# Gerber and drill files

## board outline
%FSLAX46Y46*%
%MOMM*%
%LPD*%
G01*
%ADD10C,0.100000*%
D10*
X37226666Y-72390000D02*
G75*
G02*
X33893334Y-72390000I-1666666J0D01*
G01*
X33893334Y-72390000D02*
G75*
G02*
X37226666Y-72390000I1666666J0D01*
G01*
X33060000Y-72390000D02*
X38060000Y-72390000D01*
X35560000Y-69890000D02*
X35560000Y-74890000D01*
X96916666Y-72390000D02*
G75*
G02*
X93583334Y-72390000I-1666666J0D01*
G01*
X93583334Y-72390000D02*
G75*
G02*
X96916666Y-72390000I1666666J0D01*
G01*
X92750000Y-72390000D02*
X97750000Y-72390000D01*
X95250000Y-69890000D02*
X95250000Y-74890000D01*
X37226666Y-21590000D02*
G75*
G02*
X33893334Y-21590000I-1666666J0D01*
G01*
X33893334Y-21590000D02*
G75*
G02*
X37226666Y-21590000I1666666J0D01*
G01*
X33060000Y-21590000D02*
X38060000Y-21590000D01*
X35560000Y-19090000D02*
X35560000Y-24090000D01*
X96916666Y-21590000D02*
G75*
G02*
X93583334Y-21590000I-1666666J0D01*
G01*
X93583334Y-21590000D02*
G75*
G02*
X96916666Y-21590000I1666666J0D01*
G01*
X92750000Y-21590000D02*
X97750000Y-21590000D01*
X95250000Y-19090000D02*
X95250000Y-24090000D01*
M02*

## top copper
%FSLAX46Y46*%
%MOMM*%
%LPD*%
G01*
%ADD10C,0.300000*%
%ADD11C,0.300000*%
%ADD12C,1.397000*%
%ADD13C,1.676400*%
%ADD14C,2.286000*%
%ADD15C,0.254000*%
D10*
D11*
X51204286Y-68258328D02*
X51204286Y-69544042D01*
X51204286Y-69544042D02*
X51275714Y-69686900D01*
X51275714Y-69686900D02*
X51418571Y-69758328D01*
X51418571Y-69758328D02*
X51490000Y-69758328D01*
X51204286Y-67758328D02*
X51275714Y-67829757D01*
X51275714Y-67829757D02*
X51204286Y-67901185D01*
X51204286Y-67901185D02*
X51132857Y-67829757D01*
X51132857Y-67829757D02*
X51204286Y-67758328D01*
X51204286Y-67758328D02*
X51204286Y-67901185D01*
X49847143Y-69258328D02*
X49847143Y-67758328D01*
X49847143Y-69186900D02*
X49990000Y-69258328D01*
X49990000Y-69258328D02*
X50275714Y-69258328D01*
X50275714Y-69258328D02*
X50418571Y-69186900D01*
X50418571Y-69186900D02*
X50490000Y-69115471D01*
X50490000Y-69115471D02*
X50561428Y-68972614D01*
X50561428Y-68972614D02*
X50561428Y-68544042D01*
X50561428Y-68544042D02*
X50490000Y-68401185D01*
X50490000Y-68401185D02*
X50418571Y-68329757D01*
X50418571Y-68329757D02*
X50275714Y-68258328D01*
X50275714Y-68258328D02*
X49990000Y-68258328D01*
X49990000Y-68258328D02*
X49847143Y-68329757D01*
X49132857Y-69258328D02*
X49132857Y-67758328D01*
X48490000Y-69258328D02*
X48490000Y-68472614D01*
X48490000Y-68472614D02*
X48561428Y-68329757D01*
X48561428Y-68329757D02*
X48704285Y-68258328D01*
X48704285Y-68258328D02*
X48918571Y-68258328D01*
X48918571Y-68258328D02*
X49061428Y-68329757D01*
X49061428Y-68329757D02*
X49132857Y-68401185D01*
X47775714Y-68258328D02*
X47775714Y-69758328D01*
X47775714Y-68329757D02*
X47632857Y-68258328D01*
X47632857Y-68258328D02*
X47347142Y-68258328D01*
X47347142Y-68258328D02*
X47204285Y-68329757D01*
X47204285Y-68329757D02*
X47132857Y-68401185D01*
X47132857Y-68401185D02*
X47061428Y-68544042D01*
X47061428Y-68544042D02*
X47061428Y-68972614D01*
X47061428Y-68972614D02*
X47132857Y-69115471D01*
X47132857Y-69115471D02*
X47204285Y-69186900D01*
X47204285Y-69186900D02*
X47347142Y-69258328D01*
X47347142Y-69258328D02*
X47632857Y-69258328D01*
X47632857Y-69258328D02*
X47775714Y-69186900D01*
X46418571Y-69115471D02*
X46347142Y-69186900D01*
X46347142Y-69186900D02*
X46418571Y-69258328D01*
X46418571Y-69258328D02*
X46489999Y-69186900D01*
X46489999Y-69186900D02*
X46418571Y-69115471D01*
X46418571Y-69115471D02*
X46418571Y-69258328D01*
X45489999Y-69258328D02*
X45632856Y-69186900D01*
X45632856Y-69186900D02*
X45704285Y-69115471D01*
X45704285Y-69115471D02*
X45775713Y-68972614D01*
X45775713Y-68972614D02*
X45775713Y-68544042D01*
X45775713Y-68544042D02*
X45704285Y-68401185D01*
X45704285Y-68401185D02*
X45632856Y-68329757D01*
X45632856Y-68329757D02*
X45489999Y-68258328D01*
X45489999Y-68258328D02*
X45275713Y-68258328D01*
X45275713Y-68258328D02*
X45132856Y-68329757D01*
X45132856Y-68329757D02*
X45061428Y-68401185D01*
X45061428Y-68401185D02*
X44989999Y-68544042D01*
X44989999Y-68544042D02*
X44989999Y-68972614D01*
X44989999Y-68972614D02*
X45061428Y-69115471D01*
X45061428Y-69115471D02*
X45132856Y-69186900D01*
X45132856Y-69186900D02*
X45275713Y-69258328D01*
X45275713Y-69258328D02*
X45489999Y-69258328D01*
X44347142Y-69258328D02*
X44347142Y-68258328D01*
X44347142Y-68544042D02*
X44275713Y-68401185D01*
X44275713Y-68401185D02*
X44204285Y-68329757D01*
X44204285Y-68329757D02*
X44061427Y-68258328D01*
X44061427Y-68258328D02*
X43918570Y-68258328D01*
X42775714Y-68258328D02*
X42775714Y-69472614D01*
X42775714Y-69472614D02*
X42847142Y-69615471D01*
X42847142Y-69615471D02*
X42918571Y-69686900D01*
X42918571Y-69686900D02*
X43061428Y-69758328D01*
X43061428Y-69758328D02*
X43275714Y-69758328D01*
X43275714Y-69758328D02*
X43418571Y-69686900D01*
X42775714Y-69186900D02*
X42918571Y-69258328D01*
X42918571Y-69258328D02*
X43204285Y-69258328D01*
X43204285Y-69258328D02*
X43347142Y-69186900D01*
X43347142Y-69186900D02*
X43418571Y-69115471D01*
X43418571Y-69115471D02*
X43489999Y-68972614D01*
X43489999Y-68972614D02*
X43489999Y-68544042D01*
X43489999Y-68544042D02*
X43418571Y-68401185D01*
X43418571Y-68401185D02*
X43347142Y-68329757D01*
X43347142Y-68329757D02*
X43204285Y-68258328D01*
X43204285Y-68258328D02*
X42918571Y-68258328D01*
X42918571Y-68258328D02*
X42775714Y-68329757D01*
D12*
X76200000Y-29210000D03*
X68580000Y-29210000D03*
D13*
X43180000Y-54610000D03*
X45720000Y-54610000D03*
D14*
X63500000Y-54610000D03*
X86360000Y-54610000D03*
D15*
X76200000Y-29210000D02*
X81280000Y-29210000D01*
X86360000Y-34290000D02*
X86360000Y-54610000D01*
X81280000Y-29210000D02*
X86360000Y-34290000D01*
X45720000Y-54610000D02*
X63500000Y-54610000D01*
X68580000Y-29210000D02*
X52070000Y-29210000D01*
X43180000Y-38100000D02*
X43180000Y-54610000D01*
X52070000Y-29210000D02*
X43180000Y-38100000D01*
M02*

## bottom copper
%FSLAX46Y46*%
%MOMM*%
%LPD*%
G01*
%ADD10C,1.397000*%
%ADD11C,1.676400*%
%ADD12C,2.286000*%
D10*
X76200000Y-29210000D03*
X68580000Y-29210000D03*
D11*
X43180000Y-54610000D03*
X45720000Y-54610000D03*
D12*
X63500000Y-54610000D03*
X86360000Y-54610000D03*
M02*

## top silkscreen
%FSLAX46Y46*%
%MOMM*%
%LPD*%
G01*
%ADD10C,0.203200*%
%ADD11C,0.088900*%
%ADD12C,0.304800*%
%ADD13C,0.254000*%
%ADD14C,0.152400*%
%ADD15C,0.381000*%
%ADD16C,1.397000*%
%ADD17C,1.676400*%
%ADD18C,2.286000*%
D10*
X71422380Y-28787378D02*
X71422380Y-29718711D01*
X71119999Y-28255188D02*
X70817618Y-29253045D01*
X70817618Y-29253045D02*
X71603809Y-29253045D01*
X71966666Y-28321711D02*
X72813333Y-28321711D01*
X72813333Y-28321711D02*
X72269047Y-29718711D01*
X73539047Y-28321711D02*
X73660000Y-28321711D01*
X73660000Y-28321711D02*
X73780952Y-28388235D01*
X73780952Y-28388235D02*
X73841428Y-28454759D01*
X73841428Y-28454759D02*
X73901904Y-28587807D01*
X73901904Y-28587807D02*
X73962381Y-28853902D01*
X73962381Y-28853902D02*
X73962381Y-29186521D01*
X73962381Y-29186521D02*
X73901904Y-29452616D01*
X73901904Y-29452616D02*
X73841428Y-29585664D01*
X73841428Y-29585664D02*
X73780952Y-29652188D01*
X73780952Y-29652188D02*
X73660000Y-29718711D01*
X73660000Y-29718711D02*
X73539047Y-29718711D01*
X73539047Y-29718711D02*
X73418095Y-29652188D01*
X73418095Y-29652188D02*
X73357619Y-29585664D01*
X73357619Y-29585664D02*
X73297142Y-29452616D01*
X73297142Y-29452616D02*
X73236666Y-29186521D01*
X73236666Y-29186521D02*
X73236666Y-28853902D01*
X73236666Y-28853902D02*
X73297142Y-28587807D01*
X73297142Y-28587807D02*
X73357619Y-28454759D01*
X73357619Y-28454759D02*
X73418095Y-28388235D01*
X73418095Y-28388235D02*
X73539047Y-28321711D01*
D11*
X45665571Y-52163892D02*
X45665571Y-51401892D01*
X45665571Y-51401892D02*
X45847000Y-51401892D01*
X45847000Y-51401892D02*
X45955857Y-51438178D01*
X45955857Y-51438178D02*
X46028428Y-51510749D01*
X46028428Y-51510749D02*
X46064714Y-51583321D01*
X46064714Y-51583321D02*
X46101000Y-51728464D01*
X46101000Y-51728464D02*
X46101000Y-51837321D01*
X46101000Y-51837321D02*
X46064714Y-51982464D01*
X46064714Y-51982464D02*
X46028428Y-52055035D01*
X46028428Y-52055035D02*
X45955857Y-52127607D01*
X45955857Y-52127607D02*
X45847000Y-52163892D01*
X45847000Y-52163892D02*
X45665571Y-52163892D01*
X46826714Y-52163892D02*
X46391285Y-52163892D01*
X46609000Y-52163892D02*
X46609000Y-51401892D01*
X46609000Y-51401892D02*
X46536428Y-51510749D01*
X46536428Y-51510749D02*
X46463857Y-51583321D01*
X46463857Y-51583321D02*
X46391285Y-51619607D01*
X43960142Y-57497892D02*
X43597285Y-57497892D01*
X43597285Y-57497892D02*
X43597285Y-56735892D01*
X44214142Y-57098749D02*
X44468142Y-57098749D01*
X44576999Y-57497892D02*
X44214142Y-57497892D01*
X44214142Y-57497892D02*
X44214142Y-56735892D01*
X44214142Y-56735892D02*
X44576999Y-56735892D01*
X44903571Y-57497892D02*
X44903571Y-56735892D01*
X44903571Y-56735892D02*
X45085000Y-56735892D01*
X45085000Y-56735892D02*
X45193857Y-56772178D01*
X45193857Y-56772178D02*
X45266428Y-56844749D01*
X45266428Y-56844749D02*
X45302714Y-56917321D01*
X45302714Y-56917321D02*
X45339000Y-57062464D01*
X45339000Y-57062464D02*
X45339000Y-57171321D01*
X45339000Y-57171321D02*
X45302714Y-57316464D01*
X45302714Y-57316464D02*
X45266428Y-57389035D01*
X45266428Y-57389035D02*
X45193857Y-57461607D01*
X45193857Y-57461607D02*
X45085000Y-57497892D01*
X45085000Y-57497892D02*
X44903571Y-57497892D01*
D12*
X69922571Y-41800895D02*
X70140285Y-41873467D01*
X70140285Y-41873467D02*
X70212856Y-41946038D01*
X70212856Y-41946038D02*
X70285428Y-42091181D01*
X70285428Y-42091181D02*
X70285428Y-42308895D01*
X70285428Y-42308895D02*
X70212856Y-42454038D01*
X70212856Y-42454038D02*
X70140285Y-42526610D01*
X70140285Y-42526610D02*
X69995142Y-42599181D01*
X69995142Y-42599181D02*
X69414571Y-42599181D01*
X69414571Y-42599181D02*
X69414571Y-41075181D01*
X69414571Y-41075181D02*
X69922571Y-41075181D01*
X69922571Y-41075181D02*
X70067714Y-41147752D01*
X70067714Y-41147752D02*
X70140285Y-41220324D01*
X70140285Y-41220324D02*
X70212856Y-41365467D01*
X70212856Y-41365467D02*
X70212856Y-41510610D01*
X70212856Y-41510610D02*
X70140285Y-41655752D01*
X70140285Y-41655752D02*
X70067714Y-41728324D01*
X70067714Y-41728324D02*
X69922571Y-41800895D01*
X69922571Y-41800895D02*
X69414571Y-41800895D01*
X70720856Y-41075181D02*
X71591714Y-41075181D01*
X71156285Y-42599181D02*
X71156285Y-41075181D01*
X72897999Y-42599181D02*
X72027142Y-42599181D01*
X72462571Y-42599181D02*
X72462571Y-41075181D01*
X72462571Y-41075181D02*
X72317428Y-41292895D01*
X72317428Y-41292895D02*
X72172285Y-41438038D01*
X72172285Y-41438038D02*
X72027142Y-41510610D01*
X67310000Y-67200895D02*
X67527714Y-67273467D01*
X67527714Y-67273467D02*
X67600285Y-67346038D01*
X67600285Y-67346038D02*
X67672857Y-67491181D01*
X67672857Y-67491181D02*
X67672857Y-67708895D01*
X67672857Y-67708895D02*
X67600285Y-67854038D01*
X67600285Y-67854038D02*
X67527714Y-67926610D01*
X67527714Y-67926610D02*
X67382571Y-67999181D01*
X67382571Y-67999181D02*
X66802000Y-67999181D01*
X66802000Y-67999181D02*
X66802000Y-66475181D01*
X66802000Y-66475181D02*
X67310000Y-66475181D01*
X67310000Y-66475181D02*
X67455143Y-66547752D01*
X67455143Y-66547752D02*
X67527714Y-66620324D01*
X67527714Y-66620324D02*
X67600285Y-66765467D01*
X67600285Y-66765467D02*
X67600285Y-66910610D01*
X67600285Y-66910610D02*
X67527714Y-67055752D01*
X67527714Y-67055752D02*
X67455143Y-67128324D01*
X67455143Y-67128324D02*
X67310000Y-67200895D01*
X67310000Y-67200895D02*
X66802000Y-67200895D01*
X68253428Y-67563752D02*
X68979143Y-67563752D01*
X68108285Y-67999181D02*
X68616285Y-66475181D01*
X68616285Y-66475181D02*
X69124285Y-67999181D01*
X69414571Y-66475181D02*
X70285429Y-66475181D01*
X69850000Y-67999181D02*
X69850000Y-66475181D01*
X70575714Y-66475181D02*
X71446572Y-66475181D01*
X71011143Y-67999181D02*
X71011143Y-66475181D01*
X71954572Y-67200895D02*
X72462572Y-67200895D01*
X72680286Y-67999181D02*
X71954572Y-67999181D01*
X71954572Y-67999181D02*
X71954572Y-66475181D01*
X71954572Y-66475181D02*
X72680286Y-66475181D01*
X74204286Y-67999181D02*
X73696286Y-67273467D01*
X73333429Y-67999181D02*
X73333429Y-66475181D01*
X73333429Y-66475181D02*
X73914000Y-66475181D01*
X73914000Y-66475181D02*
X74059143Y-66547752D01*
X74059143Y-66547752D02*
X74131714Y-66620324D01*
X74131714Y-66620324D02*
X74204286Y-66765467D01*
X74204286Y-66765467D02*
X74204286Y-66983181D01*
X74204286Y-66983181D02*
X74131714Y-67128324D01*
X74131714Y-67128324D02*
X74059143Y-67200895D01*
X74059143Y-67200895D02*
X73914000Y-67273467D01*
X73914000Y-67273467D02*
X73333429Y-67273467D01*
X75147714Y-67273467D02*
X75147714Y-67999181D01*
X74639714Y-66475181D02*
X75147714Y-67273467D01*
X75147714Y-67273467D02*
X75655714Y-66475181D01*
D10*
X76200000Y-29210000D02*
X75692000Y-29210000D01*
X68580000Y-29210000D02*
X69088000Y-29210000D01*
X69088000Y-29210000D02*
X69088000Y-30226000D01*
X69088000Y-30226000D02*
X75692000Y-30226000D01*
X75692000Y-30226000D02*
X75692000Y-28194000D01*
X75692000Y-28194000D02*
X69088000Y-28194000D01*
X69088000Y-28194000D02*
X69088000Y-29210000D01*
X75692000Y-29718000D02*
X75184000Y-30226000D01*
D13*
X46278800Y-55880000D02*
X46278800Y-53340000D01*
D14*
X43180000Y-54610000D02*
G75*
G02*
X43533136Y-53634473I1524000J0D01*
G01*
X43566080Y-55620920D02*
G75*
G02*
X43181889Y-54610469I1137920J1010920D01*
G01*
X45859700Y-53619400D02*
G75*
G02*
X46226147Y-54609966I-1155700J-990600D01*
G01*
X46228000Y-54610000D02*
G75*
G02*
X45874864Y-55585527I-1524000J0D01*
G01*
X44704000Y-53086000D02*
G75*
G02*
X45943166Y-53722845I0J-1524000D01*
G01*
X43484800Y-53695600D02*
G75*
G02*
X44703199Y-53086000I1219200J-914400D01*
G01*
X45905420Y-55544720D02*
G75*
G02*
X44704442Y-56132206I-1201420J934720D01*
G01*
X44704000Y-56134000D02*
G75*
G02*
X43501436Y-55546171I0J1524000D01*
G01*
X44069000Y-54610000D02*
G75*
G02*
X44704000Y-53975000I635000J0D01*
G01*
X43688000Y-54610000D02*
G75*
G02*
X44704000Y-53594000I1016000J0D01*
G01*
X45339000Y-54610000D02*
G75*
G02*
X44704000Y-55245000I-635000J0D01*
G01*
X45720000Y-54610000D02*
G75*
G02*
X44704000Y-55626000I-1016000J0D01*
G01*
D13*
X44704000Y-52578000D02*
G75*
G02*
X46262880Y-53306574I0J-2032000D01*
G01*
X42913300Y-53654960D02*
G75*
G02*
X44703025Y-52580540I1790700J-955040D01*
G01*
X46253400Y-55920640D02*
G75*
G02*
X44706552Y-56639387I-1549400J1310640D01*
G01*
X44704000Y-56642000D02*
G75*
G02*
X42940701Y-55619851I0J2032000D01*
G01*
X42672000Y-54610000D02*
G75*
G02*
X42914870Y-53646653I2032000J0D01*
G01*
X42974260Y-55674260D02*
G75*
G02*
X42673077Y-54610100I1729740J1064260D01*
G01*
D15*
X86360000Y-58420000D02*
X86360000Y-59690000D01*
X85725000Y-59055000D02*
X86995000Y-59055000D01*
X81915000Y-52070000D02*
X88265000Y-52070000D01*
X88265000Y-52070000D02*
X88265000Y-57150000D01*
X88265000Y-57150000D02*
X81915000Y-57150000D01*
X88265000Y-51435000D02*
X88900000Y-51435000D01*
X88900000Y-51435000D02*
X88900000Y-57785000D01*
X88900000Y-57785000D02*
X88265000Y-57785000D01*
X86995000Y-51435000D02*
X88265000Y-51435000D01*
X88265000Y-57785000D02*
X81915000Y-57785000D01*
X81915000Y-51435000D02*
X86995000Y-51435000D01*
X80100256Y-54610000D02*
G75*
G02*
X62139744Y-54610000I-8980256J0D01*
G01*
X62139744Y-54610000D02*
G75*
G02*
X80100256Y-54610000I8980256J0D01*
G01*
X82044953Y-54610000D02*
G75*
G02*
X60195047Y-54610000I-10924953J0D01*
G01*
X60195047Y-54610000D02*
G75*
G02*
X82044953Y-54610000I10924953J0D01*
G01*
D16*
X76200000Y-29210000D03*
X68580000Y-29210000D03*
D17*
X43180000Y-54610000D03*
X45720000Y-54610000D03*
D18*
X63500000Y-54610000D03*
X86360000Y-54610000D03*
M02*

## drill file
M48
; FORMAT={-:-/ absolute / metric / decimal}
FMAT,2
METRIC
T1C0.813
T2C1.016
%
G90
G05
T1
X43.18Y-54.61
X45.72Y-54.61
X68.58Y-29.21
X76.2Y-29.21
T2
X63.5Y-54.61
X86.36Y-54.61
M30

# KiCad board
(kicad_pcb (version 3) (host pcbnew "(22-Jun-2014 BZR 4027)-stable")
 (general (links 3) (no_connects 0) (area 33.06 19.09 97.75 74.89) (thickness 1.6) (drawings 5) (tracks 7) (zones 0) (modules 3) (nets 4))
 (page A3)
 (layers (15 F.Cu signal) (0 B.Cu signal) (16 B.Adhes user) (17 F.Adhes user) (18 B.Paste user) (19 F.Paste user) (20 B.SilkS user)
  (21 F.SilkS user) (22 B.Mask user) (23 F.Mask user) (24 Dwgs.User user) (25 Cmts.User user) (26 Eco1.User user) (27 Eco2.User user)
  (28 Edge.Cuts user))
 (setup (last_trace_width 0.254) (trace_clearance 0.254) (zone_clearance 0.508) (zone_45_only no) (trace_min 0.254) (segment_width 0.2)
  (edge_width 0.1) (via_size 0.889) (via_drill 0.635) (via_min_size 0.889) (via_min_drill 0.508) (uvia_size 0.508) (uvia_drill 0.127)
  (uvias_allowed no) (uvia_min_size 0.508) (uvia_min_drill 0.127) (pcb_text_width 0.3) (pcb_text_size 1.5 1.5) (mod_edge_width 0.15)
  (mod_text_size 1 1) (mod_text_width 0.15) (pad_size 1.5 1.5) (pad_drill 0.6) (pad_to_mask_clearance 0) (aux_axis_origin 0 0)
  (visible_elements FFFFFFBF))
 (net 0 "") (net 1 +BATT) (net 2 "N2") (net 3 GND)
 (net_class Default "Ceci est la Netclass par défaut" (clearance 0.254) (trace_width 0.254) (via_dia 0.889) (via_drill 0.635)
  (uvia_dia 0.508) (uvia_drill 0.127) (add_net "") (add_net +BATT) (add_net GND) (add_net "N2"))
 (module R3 (layer F.Cu) (at 72.39 29.21 180) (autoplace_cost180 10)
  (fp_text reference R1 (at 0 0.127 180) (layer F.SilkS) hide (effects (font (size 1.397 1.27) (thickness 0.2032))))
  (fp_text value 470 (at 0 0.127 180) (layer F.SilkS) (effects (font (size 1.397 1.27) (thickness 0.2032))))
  (fp_line (start -3.81 0) (end -3.302 0) (layer F.SilkS) (width 0.2032))
  (fp_line (start 3.81 0) (end 3.302 0) (layer F.SilkS) (width 0.2032))
  (fp_line (start 3.302 0) (end 3.302 -1.016) (layer F.SilkS) (width 0.2032))
  (fp_line (start 3.302 -1.016) (end -3.302 -1.016) (layer F.SilkS) (width 0.2032))
  (fp_line (start -3.302 -1.016) (end -3.302 1.016) (layer F.SilkS) (width 0.2032))
  (fp_line (start -3.302 1.016) (end 3.302 1.016) (layer F.SilkS) (width 0.2032))
  (fp_line (start 3.302 1.016) (end 3.302 0) (layer F.SilkS) (width 0.2032))
  (fp_line (start -3.302 -0.508) (end -2.794 -1.016) (layer F.SilkS) (width 0.2032))
  (pad 1 thru_hole circle (at -3.81 0 180) (size 1.397 1.397) (drill 0.8128) (layers *.Cu *.Mask F.SilkS) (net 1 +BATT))
  (pad 2 thru_hole circle (at 3.81 0 180) (size 1.397 1.397) (drill 0.8128) (layers *.Cu *.Mask F.SilkS) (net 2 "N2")))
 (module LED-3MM (layer F.Cu) (at 44.45 54.61)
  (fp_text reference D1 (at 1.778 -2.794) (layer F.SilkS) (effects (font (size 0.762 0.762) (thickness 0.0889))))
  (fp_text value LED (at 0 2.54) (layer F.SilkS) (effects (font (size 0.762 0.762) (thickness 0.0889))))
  (fp_line (start 1.8288 1.27) (end 1.8288 -1.27) (layer F.SilkS) (width 0.254))
  (fp_arc (start 0.254 0) (end -1.27 0) (angle 39.8) (layer F.SilkS) (width 0.1524))
  (fp_arc (start 0.254 0) (end -0.88392 1.01092) (angle 41.6) (layer F.SilkS) (width 0.1524))
  (fp_arc (start 0.254 0) (end 1.4097 -0.9906) (angle 40.6) (layer F.SilkS) (width 0.1524))
  (fp_arc (start 0.254 0) (end 1.778 0) (angle 39.8) (layer F.SilkS) (width 0.1524))
  (fp_arc (start 0.254 0) (end 0.254 -1.524) (angle 54.4) (layer F.SilkS) (width 0.1524))
  (fp_arc (start 0.254 0) (end -0.9652 -0.9144) (angle 53.1) (layer F.SilkS) (width 0.1524))
  (fp_arc (start 0.254 0) (end 1.45542 0.93472) (angle 52.1) (layer F.SilkS) (width 0.1524))
  (fp_arc (start 0.254 0) (end 0.254 1.524) (angle 52.1) (layer F.SilkS) (width 0.1524))
  (fp_arc (start 0.254 0) (end -0.381 0) (angle 90) (layer F.SilkS) (width 0.1524))
  (fp_arc (start 0.254 0) (end -0.762 0) (angle 90) (layer F.SilkS) (width 0.1524))
  (fp_arc (start 0.254 0) (end 0.889 0) (angle 90) (layer F.SilkS) (width 0.1524))
  (fp_arc (start 0.254 0) (end 1.27 0) (angle 90) (layer F.SilkS) (width 0.1524))
  (fp_arc (start 0.254 0) (end 0.254 -2.032) (angle 50.1) (layer F.SilkS) (width 0.254))
  (fp_arc (start 0.254 0) (end -1.5367 -0.95504) (angle 61.9) (layer F.SilkS) (width 0.254))
  (fp_arc (start 0.254 0) (end 1.8034 1.31064) (angle 49.7) (layer F.SilkS) (width 0.254))
  (fp_arc (start 0.254 0) (end 0.254 2.032) (angle 60.2) (layer F.SilkS) (width 0.254))
  (fp_arc (start 0.254 0) (end -1.778 0) (angle 28.3) (layer F.SilkS) (width 0.254))
  (fp_arc (start 0.254 0) (end -1.47574 1.06426) (angle 31.6) (layer F.SilkS) (width 0.254))
  (pad 1 thru_hole circle (at -1.27 0) (size 1.6764 1.6764) (drill 0.8128) (layers *.Cu *.Mask F.SilkS) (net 2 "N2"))
  (pad 2 thru_hole circle (at 1.27 0) (size 1.6764 1.6764) (drill 0.8128) (layers *.Cu *.Mask F.SilkS) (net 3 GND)))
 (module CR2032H (layer F.Cu) (at 71.12 54.61)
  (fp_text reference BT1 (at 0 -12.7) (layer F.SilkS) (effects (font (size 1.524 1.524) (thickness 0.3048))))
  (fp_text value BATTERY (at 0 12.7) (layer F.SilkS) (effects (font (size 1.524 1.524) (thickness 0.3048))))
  (fp_line (start 15.24 3.81) (end 15.24 5.08) (layer F.SilkS) (width 0.381))
  (fp_line (start 14.605 4.445) (end 15.875 4.445) (layer F.SilkS) (width 0.381))
  (fp_line (start 10.795 -2.54) (end 17.145 -2.54) (layer F.SilkS) (width 0.381))
  (fp_line (start 17.145 -2.54) (end 17.145 2.54) (layer F.SilkS) (width 0.381))
  (fp_line (start 17.145 2.54) (end 10.795 2.54) (layer F.SilkS) (width 0.381))
  (fp_line (start 17.145 -3.175) (end 17.78 -3.175) (layer F.SilkS) (width 0.381))
  (fp_line (start 17.78 -3.175) (end 17.78 3.175) (layer F.SilkS) (width 0.381))
  (fp_line (start 17.78 3.175) (end 17.145 3.175) (layer F.SilkS) (width 0.381))
  (fp_line (start 15.875 -3.175) (end 17.145 -3.175) (layer F.SilkS) (width 0.381))
  (fp_line (start 17.145 3.175) (end 10.795 3.175) (layer F.SilkS) (width 0.381))
  (fp_line (start 10.795 -3.175) (end 15.875 -3.175) (layer F.SilkS) (width 0.381))
  (fp_circle (center 0 0) (end -1.27 -8.89) (layer F.SilkS) (width 0.381))
  (fp_circle (center 0 0) (end 6.35 8.89) (layer F.SilkS) (width 0.381))
  (pad 2 thru_hole circle (at -7.62 0) (size 2.286 2.286) (drill 1.016) (layers *.Cu *.Mask F.SilkS) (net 3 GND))
  (pad 1 thru_hole circle (at 15.24 0) (size 2.286 2.286) (drill 1.016) (layers *.Cu *.Mask F.SilkS) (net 1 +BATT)))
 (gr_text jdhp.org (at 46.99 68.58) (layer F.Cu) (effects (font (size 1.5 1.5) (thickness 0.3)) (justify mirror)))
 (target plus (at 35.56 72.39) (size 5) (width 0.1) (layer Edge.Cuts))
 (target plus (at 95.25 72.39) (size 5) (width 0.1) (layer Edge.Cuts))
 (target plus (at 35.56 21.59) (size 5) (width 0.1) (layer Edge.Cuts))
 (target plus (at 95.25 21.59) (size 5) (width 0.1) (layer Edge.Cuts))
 (segment (start 76.2 29.21) (end 81.28 29.21) (width 0.254) (layer F.Cu) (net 1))
 (segment (start 86.36 34.29) (end 86.36 54.61) (width 0.254) (layer F.Cu) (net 1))
 (segment (start 81.28 29.21) (end 86.36 34.29) (width 0.254) (layer F.Cu) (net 1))
 (segment (start 45.72 54.61) (end 63.5 54.61) (width 0.254) (layer F.Cu) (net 3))
 (segment (start 68.58 29.21) (end 52.07 29.21) (width 0.254) (layer F.Cu) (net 2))
 (segment (start 43.18 38.1) (end 43.18 54.61) (width 0.254) (layer F.Cu) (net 2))
 (segment (start 52.07 29.21) (end 43.18 38.1) (width 0.254) (layer F.Cu) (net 2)))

